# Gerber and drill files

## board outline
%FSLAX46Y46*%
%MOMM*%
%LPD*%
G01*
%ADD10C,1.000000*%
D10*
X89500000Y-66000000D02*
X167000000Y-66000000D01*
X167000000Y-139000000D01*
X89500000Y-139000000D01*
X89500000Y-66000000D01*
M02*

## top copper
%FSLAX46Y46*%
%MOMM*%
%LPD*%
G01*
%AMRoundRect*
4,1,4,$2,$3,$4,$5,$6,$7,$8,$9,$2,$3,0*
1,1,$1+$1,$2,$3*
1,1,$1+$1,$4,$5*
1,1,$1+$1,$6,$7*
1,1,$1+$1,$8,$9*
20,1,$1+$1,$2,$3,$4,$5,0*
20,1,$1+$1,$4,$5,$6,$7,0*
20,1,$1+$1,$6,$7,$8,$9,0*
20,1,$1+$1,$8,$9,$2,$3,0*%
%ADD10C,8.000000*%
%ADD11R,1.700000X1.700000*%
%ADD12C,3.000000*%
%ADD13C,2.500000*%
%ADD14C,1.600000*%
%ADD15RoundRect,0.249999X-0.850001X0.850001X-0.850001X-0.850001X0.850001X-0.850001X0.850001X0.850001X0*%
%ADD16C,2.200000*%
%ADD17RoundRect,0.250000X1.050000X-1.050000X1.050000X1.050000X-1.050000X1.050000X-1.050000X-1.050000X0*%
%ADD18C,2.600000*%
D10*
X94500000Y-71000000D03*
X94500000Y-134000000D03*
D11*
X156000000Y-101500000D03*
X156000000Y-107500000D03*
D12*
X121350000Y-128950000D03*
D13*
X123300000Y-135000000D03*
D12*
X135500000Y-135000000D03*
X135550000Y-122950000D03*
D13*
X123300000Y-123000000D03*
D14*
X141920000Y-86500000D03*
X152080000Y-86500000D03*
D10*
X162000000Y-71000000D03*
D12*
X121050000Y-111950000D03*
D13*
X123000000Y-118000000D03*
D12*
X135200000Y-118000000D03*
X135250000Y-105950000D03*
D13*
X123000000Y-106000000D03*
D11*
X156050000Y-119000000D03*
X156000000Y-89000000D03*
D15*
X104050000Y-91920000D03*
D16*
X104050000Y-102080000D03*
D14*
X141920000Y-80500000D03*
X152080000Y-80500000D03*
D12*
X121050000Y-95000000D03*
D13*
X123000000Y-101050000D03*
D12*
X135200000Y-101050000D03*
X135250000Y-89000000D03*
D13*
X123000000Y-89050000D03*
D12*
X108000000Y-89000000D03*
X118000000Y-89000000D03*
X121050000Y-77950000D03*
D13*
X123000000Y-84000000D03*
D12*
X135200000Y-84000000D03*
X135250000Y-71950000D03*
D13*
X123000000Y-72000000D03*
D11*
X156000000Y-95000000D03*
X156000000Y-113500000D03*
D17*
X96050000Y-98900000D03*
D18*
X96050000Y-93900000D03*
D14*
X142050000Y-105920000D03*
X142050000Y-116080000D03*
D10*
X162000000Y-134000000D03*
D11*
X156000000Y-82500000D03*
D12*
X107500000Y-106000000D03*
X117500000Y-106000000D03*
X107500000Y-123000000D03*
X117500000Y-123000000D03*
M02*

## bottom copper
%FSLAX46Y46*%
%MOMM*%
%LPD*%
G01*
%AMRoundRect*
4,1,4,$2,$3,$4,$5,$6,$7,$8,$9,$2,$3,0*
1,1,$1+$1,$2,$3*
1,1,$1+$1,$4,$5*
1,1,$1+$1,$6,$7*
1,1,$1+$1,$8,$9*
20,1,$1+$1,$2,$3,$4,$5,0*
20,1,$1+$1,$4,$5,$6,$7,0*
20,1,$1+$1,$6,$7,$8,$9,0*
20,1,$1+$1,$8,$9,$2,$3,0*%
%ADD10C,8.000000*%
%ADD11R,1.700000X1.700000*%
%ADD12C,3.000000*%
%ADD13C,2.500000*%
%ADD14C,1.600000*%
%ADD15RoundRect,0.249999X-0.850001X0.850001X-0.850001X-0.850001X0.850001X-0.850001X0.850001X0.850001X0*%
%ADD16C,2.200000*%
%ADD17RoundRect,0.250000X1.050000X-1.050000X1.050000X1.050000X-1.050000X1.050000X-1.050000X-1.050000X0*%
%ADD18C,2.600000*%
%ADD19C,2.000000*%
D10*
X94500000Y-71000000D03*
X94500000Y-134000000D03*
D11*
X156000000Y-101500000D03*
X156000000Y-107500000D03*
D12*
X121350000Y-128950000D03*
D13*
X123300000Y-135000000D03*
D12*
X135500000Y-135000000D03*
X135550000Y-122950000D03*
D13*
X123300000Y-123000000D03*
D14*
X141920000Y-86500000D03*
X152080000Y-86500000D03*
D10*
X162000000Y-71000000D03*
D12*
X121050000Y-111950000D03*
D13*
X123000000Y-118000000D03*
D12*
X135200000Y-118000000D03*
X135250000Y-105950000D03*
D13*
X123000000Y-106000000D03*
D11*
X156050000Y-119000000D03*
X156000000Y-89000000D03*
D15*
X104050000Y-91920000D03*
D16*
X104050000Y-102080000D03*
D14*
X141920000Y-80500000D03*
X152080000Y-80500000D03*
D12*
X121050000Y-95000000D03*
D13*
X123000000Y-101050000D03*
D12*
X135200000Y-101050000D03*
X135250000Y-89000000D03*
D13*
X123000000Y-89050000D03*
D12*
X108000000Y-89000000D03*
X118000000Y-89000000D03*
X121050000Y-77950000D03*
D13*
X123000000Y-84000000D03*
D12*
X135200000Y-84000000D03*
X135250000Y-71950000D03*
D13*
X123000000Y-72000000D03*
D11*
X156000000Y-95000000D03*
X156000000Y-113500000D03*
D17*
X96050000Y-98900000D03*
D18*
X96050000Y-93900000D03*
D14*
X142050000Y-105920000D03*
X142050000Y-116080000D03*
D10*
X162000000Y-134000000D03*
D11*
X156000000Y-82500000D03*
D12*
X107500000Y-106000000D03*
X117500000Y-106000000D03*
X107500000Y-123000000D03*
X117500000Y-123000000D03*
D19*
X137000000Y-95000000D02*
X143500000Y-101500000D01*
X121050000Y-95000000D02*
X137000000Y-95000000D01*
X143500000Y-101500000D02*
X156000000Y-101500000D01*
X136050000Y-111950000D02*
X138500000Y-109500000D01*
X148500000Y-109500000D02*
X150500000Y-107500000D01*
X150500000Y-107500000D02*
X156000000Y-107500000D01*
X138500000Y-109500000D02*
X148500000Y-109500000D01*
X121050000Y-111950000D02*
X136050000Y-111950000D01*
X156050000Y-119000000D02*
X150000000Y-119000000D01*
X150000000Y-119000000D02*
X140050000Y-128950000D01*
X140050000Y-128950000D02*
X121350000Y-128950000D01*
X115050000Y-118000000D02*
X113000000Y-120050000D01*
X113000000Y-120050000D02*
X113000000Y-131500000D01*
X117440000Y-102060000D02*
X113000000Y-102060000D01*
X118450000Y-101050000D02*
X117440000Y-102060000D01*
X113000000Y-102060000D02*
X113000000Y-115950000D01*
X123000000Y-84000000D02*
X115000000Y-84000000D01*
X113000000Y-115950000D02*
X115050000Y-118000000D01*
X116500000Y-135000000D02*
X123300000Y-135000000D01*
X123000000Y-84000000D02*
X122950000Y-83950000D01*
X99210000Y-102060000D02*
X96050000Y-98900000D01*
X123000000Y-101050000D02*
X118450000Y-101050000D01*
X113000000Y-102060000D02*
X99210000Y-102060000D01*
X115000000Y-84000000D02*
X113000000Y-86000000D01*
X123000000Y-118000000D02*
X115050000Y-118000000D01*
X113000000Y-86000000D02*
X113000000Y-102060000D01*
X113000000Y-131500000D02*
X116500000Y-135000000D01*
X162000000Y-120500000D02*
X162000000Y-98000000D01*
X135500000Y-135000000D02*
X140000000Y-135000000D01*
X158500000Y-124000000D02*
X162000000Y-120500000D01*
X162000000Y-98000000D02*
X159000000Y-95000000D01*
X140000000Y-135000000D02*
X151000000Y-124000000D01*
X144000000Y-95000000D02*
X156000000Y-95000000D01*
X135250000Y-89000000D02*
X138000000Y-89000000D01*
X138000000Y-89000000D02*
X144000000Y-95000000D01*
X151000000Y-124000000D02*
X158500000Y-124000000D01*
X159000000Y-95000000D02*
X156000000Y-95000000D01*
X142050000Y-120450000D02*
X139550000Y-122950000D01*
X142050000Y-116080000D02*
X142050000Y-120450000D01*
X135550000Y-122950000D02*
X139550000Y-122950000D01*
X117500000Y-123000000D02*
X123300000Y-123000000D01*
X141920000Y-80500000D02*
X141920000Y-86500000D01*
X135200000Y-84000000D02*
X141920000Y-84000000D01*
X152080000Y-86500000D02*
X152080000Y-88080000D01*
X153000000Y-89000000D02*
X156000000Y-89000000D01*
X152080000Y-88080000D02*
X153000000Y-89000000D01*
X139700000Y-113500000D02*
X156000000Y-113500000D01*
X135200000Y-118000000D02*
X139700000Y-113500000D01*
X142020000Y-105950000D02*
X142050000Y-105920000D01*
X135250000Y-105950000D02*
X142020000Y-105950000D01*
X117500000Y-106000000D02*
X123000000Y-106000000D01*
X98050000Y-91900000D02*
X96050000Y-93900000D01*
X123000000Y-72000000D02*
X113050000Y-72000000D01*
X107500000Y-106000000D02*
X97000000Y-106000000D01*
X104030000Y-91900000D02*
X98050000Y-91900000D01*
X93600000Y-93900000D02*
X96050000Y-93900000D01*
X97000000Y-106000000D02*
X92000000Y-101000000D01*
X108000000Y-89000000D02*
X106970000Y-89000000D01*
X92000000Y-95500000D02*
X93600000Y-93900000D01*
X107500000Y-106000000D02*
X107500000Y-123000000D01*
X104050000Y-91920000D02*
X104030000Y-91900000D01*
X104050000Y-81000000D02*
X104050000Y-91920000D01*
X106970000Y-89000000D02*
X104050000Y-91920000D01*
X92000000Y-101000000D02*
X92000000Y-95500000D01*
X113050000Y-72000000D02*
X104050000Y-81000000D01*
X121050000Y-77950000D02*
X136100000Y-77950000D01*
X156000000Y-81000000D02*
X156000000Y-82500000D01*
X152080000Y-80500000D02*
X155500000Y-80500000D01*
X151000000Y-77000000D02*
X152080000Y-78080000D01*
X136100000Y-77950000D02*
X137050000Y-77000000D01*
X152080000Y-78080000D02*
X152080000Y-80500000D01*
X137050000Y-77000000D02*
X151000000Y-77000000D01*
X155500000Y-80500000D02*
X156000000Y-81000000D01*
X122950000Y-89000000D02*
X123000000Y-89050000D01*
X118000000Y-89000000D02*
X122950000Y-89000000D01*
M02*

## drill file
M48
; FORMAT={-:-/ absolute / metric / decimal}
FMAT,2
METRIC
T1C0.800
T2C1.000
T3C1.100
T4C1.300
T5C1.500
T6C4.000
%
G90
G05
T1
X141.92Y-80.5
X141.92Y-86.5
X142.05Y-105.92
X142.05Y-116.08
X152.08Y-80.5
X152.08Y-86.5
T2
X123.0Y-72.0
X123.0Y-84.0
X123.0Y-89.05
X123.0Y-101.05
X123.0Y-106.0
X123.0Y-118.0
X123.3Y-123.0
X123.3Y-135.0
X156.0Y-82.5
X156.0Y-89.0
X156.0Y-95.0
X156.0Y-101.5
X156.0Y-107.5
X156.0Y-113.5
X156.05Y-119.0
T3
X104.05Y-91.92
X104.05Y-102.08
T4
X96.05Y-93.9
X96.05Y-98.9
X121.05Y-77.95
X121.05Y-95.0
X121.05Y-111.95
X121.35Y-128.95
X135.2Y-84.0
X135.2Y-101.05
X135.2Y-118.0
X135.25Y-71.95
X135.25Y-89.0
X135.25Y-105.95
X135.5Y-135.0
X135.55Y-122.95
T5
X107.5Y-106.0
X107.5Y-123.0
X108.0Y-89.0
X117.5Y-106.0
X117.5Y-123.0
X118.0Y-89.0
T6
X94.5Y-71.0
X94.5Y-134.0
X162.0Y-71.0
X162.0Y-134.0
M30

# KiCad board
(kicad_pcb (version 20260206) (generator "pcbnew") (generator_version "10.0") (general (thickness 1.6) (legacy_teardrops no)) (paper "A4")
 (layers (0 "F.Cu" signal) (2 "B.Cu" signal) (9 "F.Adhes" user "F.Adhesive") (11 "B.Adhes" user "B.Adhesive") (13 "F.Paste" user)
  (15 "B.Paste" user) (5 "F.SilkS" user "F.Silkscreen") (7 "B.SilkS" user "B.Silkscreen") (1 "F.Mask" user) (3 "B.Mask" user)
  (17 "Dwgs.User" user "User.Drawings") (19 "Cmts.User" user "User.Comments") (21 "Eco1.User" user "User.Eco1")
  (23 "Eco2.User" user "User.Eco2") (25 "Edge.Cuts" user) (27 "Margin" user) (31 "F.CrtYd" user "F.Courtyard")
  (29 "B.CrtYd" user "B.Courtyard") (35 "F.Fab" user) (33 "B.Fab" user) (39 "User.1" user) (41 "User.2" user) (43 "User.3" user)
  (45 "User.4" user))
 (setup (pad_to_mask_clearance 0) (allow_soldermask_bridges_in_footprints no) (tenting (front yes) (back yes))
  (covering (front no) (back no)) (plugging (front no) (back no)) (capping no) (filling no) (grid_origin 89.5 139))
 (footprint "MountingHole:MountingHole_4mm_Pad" (layer "F.Cu") (at 94.5 71)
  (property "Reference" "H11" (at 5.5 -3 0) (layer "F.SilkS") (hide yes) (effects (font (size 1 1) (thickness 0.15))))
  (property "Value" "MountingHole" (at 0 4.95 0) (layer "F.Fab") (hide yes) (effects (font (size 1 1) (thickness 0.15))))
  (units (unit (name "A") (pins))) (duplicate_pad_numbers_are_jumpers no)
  (pad "1" thru_hole circle (at 0 0) (size 8 8) (drill 4) (layers "*.Cu" "*.Mask") (remove_unused_layers no) (zone_connect 2)))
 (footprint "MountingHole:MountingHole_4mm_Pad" (layer "F.Cu") (at 94.5 134)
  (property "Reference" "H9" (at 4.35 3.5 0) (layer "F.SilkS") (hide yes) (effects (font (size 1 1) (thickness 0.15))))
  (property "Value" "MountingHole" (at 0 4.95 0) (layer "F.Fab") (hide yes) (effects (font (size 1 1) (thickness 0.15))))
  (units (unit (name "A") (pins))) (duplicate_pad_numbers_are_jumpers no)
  (pad "1" thru_hole circle (at 0 0) (size 8 8) (drill 4) (layers "*.Cu" "*.Mask") (remove_unused_layers no) (zone_connect 2)))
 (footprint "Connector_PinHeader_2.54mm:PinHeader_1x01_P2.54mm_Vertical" (layer "F.Cu") (at 156 101.5)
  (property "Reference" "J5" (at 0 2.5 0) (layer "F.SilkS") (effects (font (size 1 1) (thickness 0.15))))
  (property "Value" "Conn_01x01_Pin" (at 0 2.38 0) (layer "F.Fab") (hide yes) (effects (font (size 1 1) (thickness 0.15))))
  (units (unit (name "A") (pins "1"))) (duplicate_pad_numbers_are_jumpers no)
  (pad "1" thru_hole rect (at 0 0) (size 1.7 1.7) (drill 1) (layers "*.Cu" "*.Mask") (remove_unused_layers no) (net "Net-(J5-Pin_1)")))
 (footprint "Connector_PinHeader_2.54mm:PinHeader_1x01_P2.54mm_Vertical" (layer "F.Cu") (at 156 107.5)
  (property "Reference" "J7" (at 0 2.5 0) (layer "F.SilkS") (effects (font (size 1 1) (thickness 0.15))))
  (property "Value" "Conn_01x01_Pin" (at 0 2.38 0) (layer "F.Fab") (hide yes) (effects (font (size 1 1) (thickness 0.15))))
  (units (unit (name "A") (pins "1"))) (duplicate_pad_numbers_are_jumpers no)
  (pad "1" thru_hole rect (at 0 0) (size 1.7 1.7) (drill 1) (layers "*.Cu" "*.Mask") (remove_unused_layers no) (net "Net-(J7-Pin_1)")))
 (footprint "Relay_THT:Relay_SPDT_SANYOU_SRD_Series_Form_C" (layer "F.Cu") (at 121.35 128.95)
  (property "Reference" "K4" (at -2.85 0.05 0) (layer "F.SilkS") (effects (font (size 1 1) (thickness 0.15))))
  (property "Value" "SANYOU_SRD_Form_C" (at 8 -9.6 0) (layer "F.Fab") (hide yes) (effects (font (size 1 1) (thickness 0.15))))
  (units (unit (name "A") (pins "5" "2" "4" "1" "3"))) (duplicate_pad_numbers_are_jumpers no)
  (pad "1" thru_hole circle (at 0 0 90) (size 3 3) (drill 1.3) (layers "*.Cu" "*.Mask") (remove_unused_layers no) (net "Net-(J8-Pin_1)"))
  (pad "2" thru_hole circle (at 1.95 6.05 90) (size 2.5 2.5) (drill 1) (layers "*.Cu" "*.Mask") (remove_unused_layers no) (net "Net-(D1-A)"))
  (pad "3" thru_hole circle (at 14.15 6.05 90) (size 3 3) (drill 1.3) (layers "*.Cu" "*.Mask") (remove_unused_layers no)
   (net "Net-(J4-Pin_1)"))
  (pad "4" thru_hole circle (at 14.2 -6 90) (size 3 3) (drill 1.3) (layers "*.Cu" "*.Mask") (remove_unused_layers no) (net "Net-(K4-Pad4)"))
  (pad "5" thru_hole circle (at 1.95 -5.95 90) (size 2.5 2.5) (drill 1) (layers "*.Cu" "*.Mask") (remove_unused_layers no)
   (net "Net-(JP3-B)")))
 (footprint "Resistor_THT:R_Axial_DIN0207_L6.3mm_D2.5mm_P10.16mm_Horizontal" (layer "F.Cu") (at 141.92 86.5)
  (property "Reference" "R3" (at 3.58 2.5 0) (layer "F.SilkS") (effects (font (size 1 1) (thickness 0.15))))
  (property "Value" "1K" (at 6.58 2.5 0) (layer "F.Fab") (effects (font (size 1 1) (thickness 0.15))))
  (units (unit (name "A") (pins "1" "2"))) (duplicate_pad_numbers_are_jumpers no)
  (pad "1" thru_hole circle (at 0 0) (size 1.6 1.6) (drill 0.8) (layers "*.Cu" "*.Mask") (remove_unused_layers no) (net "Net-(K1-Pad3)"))
  (pad "2" thru_hole circle (at 10.16 0) (size 1.6 1.6) (drill 0.8) (layers "*.Cu" "*.Mask") (remove_unused_layers no)
   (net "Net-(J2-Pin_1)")))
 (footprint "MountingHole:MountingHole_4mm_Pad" (layer "F.Cu") (at 162 71)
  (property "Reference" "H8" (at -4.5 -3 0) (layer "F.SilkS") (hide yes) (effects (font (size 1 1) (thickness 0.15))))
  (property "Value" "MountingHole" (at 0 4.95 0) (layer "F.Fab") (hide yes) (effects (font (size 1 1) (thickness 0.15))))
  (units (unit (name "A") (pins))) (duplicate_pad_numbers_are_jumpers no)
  (pad "1" thru_hole circle (at 0 0) (size 8 8) (drill 4) (layers "*.Cu" "*.Mask") (remove_unused_layers no) (zone_connect 2)))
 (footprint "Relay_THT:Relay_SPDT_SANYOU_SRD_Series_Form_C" (layer "F.Cu") (at 121.05 111.95)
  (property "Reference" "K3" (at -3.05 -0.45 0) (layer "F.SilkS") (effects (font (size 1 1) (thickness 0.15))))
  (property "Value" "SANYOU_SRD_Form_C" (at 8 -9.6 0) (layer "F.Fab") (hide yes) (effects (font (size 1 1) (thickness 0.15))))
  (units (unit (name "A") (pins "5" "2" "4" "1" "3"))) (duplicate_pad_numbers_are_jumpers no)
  (pad "1" thru_hole circle (at 0 0 90) (size 3 3) (drill 1.3) (layers "*.Cu" "*.Mask") (remove_unused_layers no) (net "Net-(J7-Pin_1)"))
  (pad "2" thru_hole circle (at 1.95 6.05 90) (size 2.5 2.5) (drill 1) (layers "*.Cu" "*.Mask") (remove_unused_layers no) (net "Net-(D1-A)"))
  (pad "3" thru_hole circle (at 14.15 6.05 90) (size 3 3) (drill 1.3) (layers "*.Cu" "*.Mask") (remove_unused_layers no)
   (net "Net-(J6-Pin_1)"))
  (pad "4" thru_hole circle (at 14.2 -6 90) (size 3 3) (drill 1.3) (layers "*.Cu" "*.Mask") (remove_unused_layers no) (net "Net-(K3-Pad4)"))
  (pad "5" thru_hole circle (at 1.95 -5.95 90) (size 2.5 2.5) (drill 1) (layers "*.Cu" "*.Mask") (remove_unused_layers no)
   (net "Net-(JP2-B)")))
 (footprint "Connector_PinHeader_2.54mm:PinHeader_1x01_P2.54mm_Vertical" (layer "F.Cu") (at 156.05 119)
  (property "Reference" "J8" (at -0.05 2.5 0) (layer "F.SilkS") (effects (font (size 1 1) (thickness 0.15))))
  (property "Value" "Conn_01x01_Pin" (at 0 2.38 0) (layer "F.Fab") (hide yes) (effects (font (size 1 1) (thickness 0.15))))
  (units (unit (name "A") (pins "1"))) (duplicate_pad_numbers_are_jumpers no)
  (pad "1" thru_hole rect (at 0 0) (size 1.7 1.7) (drill 1) (layers "*.Cu" "*.Mask") (remove_unused_layers no) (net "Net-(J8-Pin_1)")))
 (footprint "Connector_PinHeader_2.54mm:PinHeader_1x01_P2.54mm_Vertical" (layer "F.Cu") (at 156 89)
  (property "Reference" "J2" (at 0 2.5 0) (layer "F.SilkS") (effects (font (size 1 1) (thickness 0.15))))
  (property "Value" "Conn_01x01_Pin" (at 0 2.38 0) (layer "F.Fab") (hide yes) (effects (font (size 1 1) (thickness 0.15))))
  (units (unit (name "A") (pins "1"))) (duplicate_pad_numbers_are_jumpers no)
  (pad "1" thru_hole rect (at 0 0) (size 1.7 1.7) (drill 1) (layers "*.Cu" "*.Mask") (remove_unused_layers no) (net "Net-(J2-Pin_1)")))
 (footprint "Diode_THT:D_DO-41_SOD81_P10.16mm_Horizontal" (layer "F.Cu") (at 104.05 91.92 -90)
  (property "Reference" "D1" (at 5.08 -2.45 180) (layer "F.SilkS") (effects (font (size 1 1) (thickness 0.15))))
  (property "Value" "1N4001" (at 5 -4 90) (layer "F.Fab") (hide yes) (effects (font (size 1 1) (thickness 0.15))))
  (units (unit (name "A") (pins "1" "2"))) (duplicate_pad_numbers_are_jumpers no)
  (pad "1" thru_hole roundrect (at 0 0 270) (size 2.2 2.2) (drill 1.1) (layers "*.Cu" "*.Mask") (remove_unused_layers no)
   (roundrect_rratio 0.113636) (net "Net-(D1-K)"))
  (pad "2" thru_hole circle (at 10.16 0 270) (size 2.2 2.2) (drill 1.1) (layers "*.Cu" "*.Mask") (remove_unused_layers no)
   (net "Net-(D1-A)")))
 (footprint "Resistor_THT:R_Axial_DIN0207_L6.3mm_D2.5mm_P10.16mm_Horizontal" (layer "F.Cu") (at 141.92 80.5)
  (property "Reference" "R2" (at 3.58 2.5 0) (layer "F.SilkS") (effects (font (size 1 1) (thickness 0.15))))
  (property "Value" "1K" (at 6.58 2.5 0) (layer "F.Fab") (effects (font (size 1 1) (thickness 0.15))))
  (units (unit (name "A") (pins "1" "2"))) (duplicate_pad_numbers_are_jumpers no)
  (pad "1" thru_hole circle (at 0 0) (size 1.6 1.6) (drill 0.8) (layers "*.Cu" "*.Mask") (remove_unused_layers no) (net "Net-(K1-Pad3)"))
  (pad "2" thru_hole circle (at 10.16 0) (size 1.6 1.6) (drill 0.8) (layers "*.Cu" "*.Mask") (remove_unused_layers no)
   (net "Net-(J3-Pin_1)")))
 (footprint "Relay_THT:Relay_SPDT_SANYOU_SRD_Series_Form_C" (layer "F.Cu") (at 121.05 95)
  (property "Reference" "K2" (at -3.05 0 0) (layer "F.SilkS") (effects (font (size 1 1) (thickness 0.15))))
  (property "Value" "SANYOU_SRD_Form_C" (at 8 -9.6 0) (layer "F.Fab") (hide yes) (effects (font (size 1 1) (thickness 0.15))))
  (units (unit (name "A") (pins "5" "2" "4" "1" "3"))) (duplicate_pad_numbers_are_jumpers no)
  (pad "1" thru_hole circle (at 0 0 90) (size 3 3) (drill 1.3) (layers "*.Cu" "*.Mask") (remove_unused_layers no) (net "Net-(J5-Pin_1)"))
  (pad "2" thru_hole circle (at 1.95 6.05 90) (size 2.5 2.5) (drill 1) (layers "*.Cu" "*.Mask") (remove_unused_layers no) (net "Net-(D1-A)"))
  (pad "3" thru_hole circle (at 14.15 6.05 90) (size 3 3) (drill 1.3) (layers "*.Cu" "*.Mask") (remove_unused_layers no)
   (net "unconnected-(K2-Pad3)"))
  (pad "4" thru_hole circle (at 14.2 -6 90) (size 3 3) (drill 1.3) (layers "*.Cu" "*.Mask") (remove_unused_layers no) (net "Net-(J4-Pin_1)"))
  (pad "5" thru_hole circle (at 1.95 -5.95 90) (size 2.5 2.5) (drill 1) (layers "*.Cu" "*.Mask") (remove_unused_layers no)
   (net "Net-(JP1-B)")))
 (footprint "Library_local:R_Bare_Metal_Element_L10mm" (layer "F.Cu") (at 108 89)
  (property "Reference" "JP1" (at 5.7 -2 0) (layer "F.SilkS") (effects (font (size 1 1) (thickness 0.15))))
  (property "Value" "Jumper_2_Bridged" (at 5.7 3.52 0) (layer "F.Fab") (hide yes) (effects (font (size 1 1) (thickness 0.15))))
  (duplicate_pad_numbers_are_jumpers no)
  (pad "1" thru_hole circle (at 0 0) (size 3 3) (drill 1.5) (layers "*.Cu" "*.Mask") (remove_unused_layers no) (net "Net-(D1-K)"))
  (pad "2" thru_hole circle (at 10 0) (size 3 3) (drill 1.5) (layers "*.Cu" "*.Mask") (remove_unused_layers no) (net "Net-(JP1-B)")))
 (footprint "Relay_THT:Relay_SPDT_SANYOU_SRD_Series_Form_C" (layer "F.Cu") (at 121.05 77.95)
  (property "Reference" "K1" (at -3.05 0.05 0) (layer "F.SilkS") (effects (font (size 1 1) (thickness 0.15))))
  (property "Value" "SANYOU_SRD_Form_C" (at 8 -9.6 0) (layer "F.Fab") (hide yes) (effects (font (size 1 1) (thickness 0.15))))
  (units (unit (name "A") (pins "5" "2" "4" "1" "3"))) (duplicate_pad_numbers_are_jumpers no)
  (pad "1" thru_hole circle (at 0 0 90) (size 3 3) (drill 1.3) (layers "*.Cu" "*.Mask") (remove_unused_layers no) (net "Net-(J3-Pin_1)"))
  (pad "2" thru_hole circle (at 1.95 6.05 90) (size 2.5 2.5) (drill 1) (layers "*.Cu" "*.Mask") (remove_unused_layers no) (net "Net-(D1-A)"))
  (pad "3" thru_hole circle (at 14.15 6.05 90) (size 3 3) (drill 1.3) (layers "*.Cu" "*.Mask") (remove_unused_layers no)
   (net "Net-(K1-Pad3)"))
  (pad "4" thru_hole circle (at 14.2 -6 90) (size 3 3) (drill 1.3) (layers "*.Cu" "*.Mask") (remove_unused_layers no)
   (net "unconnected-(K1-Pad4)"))
  (pad "5" thru_hole circle (at 1.95 -5.95 90) (size 2.5 2.5) (drill 1) (layers "*.Cu" "*.Mask") (remove_unused_layers no)
   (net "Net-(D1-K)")))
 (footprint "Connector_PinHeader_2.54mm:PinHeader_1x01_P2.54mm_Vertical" (layer "F.Cu") (at 156 95)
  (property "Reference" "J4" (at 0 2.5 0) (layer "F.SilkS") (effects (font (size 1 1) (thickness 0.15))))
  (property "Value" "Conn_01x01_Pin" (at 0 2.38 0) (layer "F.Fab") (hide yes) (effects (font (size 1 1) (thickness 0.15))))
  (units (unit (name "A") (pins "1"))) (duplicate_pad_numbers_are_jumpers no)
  (pad "1" thru_hole rect (at 0 0) (size 1.7 1.7) (drill 1) (layers "*.Cu" "*.Mask") (remove_unused_layers no) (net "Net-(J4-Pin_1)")))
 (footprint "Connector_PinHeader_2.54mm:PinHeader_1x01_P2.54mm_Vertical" (layer "F.Cu") (at 156 113.5)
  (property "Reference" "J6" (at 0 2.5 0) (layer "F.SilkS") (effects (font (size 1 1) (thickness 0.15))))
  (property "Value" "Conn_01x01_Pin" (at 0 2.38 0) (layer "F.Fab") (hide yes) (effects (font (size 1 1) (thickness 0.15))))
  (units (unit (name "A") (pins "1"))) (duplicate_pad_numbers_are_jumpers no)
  (pad "1" thru_hole rect (at 0 0) (size 1.7 1.7) (drill 1) (layers "*.Cu" "*.Mask") (remove_unused_layers no) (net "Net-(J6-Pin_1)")))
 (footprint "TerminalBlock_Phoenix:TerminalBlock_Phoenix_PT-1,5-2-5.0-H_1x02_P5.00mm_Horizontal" (layer "F.Cu") (at 96.05 98.9 90)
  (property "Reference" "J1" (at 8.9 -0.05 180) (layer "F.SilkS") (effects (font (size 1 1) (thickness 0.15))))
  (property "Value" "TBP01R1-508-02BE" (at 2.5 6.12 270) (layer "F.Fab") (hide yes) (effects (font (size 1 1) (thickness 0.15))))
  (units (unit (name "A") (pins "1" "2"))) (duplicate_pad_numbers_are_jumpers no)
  (pad "1" thru_hole roundrect (at 0 0 90) (size 2.6 2.6) (drill 1.3) (layers "*.Cu" "*.Mask") (remove_unused_layers no)
   (roundrect_rratio 0.096154) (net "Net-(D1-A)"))
  (pad "2" thru_hole circle (at 5 0 90) (size 2.6 2.6) (drill 1.3) (layers "*.Cu" "*.Mask") (remove_unused_layers no) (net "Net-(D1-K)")))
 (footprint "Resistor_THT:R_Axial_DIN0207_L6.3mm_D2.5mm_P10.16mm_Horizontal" (layer "F.Cu") (at 142.05 105.92 -90)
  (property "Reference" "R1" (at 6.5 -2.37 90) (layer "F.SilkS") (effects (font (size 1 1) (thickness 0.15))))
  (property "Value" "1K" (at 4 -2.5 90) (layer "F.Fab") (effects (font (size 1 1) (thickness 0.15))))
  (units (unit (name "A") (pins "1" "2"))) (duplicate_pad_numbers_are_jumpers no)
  (pad "1" thru_hole circle (at 0 0 270) (size 1.6 1.6) (drill 0.8) (layers "*.Cu" "*.Mask") (remove_unused_layers no) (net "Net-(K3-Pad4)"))
  (pad "2" thru_hole circle (at 10.16 0 270) (size 1.6 1.6) (drill 0.8) (layers "*.Cu" "*.Mask") (remove_unused_layers no)
   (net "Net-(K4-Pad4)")))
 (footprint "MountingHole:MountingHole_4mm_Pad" (layer "F.Cu") (at 162 134)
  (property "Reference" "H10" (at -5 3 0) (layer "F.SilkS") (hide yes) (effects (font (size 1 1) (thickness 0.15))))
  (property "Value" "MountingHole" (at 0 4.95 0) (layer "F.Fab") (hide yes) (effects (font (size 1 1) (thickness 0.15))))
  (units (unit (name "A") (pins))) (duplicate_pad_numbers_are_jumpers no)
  (pad "1" thru_hole circle (at 0 0) (size 8 8) (drill 4) (layers "*.Cu" "*.Mask") (remove_unused_layers no) (zone_connect 2)))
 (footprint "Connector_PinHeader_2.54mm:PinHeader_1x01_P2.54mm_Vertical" (layer "F.Cu") (at 156 82.5)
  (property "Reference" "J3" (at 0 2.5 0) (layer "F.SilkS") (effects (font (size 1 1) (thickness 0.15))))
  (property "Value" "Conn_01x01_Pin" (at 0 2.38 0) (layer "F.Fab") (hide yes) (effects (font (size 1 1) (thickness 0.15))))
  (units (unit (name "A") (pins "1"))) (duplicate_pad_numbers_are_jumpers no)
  (pad "1" thru_hole rect (at 0 0) (size 1.7 1.7) (drill 1) (layers "*.Cu" "*.Mask") (remove_unused_layers no) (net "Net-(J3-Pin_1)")))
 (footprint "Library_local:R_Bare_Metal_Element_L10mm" (layer "F.Cu") (at 107.5 106)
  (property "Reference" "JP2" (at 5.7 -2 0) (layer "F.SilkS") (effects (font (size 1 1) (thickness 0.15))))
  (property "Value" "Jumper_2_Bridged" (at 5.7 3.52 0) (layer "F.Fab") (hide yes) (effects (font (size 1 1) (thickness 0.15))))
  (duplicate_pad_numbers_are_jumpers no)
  (pad "1" thru_hole circle (at 0 0) (size 3 3) (drill 1.5) (layers "*.Cu" "*.Mask") (remove_unused_layers no) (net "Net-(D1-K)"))
  (pad "2" thru_hole circle (at 10 0) (size 3 3) (drill 1.5) (layers "*.Cu" "*.Mask") (remove_unused_layers no) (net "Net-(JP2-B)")))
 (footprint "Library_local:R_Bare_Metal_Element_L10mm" (layer "F.Cu") (at 107.5 123)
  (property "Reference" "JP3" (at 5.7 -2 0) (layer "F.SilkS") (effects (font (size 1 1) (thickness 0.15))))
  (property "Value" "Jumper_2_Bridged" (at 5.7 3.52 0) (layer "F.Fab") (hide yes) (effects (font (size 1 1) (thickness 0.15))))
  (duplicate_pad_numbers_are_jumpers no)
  (pad "1" thru_hole circle (at 0 0) (size 3 3) (drill 1.5) (layers "*.Cu" "*.Mask") (remove_unused_layers no) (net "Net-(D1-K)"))
  (pad "2" thru_hole circle (at 10 0) (size 3 3) (drill 1.5) (layers "*.Cu" "*.Mask") (remove_unused_layers no) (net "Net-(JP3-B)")))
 (gr_rect (start 89.5 66) (end 167 139) (stroke (width 1) (type solid)) (fill no) (locked yes) (layer "Edge.Cuts"))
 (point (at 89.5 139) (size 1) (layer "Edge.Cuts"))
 (segment (start 137 95) (end 143.5 101.5) (width 2) (layer "B.Cu") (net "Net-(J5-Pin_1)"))
 (segment (start 121.05 95) (end 137 95) (width 2) (layer "B.Cu") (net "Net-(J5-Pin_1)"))
 (segment (start 143.5 101.5) (end 156 101.5) (width 2) (layer "B.Cu") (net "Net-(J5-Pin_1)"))
 (segment (start 136.05 111.95) (end 138.5 109.5) (width 2) (layer "B.Cu") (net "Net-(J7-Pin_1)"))
 (segment (start 148.5 109.5) (end 150.5 107.5) (width 2) (layer "B.Cu") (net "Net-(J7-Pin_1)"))
 (segment (start 150.5 107.5) (end 156 107.5) (width 2) (layer "B.Cu") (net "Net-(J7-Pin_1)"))
 (segment (start 138.5 109.5) (end 148.5 109.5) (width 2) (layer "B.Cu") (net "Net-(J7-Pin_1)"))
 (segment (start 121.05 111.95) (end 136.05 111.95) (width 2) (layer "B.Cu") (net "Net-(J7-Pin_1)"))
 (segment (start 156.05 119) (end 150 119) (width 2) (layer "B.Cu") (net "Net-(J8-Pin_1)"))
 (segment (start 150 119) (end 140.05 128.95) (width 2) (layer "B.Cu") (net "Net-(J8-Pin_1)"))
 (segment (start 140.05 128.95) (end 121.35 128.95) (width 2) (layer "B.Cu") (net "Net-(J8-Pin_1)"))
 (segment (start 115.05 118) (end 113 120.05) (width 2) (layer "B.Cu") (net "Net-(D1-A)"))
 (segment (start 113 120.05) (end 113 131.5) (width 2) (layer "B.Cu") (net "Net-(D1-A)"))
 (segment (start 117.44 102.06) (end 113 102.06) (width 2) (layer "B.Cu") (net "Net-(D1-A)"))
 (segment (start 118.45 101.05) (end 117.44 102.06) (width 2) (layer "B.Cu") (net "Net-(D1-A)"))
 (segment (start 113 102.06) (end 113 115.95) (width 2) (layer "B.Cu") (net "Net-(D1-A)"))
 (segment (start 123 84) (end 115 84) (width 2) (layer "B.Cu") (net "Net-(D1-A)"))
 (segment (start 113 115.95) (end 115.05 118) (width 2) (layer "B.Cu") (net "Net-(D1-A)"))
 (segment (start 116.5 135) (end 123.3 135) (width 2) (layer "B.Cu") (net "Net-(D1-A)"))
 (segment (start 123 84) (end 122.95 83.95) (width 2) (layer "B.Cu") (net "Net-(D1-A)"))
 (segment (start 99.21 102.06) (end 96.05 98.9) (width 2) (layer "B.Cu") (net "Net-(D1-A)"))
 (segment (start 123 101.05) (end 118.45 101.05) (width 2) (layer "B.Cu") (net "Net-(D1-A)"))
 (segment (start 113 102.06) (end 99.21 102.06) (width 2) (layer "B.Cu") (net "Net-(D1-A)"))
 (segment (start 115 84) (end 113 86) (width 2) (layer "B.Cu") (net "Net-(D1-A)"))
 (segment (start 123 118) (end 115.05 118) (width 2) (layer "B.Cu") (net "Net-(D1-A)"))
 (segment (start 113 86) (end 113 102.06) (width 2) (layer "B.Cu") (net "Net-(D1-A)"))
 (segment (start 113 131.5) (end 116.5 135) (width 2) (layer "B.Cu") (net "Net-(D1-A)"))
 (segment (start 162 120.5) (end 162 98) (width 2) (layer "B.Cu") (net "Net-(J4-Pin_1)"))
 (segment (start 135.5 135) (end 140 135) (width 2) (layer "B.Cu") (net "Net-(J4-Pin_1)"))
 (segment (start 158.5 124) (end 162 120.5) (width 2) (layer "B.Cu") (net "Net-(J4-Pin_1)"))
 (segment (start 162 98) (end 159 95) (width 2) (layer "B.Cu") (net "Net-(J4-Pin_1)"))
 (segment (start 140 135) (end 151 124) (width 2) (layer "B.Cu") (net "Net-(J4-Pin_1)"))
 (segment (start 144 95) (end 156 95) (width 2) (layer "B.Cu") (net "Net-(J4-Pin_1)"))
 (segment (start 135.25 89) (end 138 89) (width 2) (layer "B.Cu") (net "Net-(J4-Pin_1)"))
 (segment (start 138 89) (end 144 95) (width 2) (layer "B.Cu") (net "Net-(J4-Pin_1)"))
 (segment (start 151 124) (end 158.5 124) (width 2) (layer "B.Cu") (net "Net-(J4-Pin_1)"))
 (segment (start 159 95) (end 156 95) (width 2) (layer "B.Cu") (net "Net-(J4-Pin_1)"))
 (segment (start 142.05 120.45) (end 139.55 122.95) (width 2) (layer "B.Cu") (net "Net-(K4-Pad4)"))
 (segment (start 142.05 116.08) (end 142.05 120.45) (width 2) (layer "B.Cu") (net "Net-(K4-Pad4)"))
 (segment (start 135.55 122.95) (end 139.55 122.95) (width 2) (layer "B.Cu") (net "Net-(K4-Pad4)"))
 (segment (start 117.5 123) (end 123.3 123) (width 2) (layer "B.Cu") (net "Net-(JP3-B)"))
 (segment (start 141.92 80.5) (end 141.92 86.5) (width 2) (layer "B.Cu") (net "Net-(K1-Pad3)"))
 (segment (start 135.2 84) (end 141.92 84) (width 2) (layer "B.Cu") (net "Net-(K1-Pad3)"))
 (segment (start 152.08 86.5) (end 152.08 88.08) (width 2) (layer "B.Cu") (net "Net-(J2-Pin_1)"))
 (segment (start 153 89) (end 156 89) (width 2) (layer "B.Cu") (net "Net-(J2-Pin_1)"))
 (segment (start 152.08 88.08) (end 153 89) (width 2) (layer "B.Cu") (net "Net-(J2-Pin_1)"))
 (segment (start 139.7 113.5) (end 156 113.5) (width 2) (layer "B.Cu") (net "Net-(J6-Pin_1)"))
 (segment (start 135.2 118) (end 139.7 113.5) (width 2) (layer "B.Cu") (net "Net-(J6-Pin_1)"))
 (segment (start 142.02 105.95) (end 142.05 105.92) (width 2) (layer "B.Cu") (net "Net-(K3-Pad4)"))
 (segment (start 135.25 105.95) (end 142.02 105.95) (width 2) (layer "B.Cu") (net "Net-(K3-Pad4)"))
 (segment (start 117.5 106) (end 123 106) (width 2) (layer "B.Cu") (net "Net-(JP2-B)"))
 (segment (start 98.05 91.9) (end 96.05 93.9) (width 2) (layer "B.Cu") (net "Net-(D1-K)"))
 (segment (start 123 72) (end 113.05 72) (width 2) (layer "B.Cu") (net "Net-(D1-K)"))
 (segment (start 107.5 106) (end 97 106) (width 2) (layer "B.Cu") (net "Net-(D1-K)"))
 (segment (start 104.03 91.9) (end 98.05 91.9) (width 2) (layer "B.Cu") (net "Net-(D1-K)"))
 (segment (start 93.6 93.9) (end 96.05 93.9) (width 2) (layer "B.Cu") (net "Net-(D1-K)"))
 (segment (start 97 106) (end 92 101) (width 2) (layer "B.Cu") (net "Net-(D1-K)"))
 (segment (start 108 89) (end 106.97 89) (width 2) (layer "B.Cu") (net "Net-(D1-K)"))
 (segment (start 92 95.5) (end 93.6 93.9) (width 2) (layer "B.Cu") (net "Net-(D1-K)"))
 (segment (start 107.5 106) (end 107.5 123) (width 2) (layer "B.Cu") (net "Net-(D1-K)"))
 (segment (start 104.05 91.92) (end 104.03 91.9) (width 2) (layer "B.Cu") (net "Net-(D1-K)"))
 (segment (start 104.05 81) (end 104.05 91.92) (width 2) (layer "B.Cu") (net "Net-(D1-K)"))
 (segment (start 106.97 89) (end 104.05 91.92) (width 2) (layer "B.Cu") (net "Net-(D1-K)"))
 (segment (start 92 101) (end 92 95.5) (width 2) (layer "B.Cu") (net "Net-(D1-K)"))
 (segment (start 113.05 72) (end 104.05 81) (width 2) (layer "B.Cu") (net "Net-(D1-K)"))
 (segment (start 121.05 77.95) (end 136.1 77.95) (width 2) (layer "B.Cu") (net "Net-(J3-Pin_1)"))
 (segment (start 156 81) (end 156 82.5) (width 2) (layer "B.Cu") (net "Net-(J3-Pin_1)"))
 (segment (start 152.08 80.5) (end 155.5 80.5) (width 2) (layer "B.Cu") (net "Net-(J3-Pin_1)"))
 (segment (start 151 77) (end 152.08 78.08) (width 2) (layer "B.Cu") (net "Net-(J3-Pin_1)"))
 (segment (start 136.1 77.95) (end 137.05 77) (width 2) (layer "B.Cu") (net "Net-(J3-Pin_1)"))
 (segment (start 152.08 78.08) (end 152.08 80.5) (width 2) (layer "B.Cu") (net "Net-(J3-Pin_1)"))
 (segment (start 137.05 77) (end 151 77) (width 2) (layer "B.Cu") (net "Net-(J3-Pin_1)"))
 (segment (start 155.5 80.5) (end 156 81) (width 2) (layer "B.Cu") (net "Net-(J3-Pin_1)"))
 (segment (start 122.95 89) (end 123 89.05) (width 2) (layer "B.Cu") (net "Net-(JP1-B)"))
 (segment (start 118 89) (end 122.95 89) (width 2) (layer "B.Cu") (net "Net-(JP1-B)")))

